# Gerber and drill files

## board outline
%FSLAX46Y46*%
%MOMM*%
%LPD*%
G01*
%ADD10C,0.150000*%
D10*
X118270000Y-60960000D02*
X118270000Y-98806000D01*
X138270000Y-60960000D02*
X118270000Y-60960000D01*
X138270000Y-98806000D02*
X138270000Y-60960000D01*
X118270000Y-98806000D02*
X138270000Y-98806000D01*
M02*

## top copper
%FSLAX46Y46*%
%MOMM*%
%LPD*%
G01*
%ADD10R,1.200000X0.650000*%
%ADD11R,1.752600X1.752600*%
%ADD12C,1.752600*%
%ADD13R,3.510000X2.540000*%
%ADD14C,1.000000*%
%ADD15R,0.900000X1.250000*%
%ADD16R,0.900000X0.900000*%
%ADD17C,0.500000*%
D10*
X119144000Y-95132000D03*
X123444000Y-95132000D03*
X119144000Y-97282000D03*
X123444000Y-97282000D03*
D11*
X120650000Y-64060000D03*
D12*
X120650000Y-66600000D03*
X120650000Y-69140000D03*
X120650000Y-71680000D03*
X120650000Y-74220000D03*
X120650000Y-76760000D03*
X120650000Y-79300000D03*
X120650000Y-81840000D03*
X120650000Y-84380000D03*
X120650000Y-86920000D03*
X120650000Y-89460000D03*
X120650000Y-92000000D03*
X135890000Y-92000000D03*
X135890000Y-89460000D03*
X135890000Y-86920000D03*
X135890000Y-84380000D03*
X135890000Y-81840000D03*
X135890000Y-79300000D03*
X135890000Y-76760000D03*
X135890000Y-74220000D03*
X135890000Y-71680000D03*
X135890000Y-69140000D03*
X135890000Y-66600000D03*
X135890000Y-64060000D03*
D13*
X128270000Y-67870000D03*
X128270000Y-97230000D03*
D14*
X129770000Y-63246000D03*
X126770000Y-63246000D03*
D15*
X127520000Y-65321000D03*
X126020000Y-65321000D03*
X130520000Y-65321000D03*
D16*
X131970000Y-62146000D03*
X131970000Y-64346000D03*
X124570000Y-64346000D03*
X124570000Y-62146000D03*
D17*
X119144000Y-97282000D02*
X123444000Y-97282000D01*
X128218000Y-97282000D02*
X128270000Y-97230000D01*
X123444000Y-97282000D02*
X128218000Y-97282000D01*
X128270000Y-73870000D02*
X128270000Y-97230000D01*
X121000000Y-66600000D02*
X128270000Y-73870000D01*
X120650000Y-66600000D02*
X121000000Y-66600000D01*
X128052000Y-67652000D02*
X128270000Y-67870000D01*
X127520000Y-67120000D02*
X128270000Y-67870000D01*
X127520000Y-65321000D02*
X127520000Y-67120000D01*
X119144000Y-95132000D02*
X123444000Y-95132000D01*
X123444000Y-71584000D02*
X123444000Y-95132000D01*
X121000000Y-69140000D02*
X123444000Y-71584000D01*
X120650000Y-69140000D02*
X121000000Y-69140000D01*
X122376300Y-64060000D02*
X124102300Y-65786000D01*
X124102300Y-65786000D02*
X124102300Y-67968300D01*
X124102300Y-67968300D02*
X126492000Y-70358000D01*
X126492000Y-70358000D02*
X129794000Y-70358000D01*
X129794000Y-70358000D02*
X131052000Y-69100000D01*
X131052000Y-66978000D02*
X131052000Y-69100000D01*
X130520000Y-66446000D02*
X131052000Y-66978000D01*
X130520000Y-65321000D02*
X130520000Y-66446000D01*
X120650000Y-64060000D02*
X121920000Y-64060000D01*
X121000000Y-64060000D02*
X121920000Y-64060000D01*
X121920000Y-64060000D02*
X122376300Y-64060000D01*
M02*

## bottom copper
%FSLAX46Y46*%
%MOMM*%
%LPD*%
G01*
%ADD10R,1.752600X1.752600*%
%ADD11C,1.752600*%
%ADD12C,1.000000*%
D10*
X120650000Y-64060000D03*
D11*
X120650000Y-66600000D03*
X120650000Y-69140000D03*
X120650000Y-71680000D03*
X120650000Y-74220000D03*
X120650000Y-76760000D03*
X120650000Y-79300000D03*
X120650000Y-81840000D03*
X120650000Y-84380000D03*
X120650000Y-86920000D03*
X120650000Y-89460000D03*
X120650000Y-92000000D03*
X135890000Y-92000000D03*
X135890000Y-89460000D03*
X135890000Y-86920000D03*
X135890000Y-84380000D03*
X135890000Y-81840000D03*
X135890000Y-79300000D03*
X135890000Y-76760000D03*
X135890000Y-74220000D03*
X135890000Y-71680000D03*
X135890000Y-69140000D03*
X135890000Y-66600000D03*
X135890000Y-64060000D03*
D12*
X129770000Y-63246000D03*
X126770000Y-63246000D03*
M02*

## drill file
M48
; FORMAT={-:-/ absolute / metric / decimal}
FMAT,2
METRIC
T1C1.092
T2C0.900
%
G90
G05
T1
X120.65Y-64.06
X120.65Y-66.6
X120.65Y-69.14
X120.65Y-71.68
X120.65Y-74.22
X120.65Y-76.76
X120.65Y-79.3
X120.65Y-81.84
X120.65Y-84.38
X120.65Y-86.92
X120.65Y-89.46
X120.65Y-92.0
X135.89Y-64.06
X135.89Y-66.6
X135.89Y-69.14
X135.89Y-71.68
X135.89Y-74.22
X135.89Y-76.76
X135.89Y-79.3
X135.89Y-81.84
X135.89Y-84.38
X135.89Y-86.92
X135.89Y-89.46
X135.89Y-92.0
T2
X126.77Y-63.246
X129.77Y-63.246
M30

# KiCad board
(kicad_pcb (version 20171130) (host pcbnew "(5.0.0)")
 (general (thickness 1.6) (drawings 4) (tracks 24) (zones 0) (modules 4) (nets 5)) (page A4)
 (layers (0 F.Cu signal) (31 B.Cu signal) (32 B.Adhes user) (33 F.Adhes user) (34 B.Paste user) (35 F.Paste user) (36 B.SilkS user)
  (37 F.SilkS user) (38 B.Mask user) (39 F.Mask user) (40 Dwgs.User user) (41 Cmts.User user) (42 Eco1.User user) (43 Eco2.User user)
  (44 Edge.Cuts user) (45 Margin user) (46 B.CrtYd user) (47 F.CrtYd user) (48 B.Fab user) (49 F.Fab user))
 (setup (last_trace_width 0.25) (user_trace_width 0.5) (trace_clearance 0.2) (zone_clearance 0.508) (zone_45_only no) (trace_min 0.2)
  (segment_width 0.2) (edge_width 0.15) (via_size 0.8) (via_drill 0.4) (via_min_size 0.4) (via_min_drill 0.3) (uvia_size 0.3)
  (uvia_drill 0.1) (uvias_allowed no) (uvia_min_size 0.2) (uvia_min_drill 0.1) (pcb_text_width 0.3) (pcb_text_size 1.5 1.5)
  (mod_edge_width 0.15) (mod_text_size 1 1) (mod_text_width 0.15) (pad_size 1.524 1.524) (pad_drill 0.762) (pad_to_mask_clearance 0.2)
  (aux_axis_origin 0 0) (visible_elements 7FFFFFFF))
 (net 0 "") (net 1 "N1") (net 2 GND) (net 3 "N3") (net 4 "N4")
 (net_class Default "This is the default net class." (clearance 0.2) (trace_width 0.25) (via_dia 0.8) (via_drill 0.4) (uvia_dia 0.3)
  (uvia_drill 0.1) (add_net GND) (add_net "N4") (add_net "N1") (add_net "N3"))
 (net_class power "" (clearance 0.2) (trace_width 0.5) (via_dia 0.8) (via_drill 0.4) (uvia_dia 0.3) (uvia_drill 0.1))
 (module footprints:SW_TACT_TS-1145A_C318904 (layer F.Cu) (at 121.294 96.207)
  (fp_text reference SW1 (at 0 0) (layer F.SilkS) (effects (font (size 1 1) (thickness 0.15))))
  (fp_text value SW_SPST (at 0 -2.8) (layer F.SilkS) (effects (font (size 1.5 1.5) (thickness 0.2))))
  (pad 1 smd rect (at -2.15 -1.075) (size 1.2 0.65) (layers F.Cu F.Paste F.Mask) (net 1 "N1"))
  (pad 1 smd rect (at 2.15 -1.075) (size 1.2 0.65) (layers F.Cu F.Paste F.Mask) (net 1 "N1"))
  (pad 2 smd rect (at -2.15 1.075) (size 1.2 0.65) (layers F.Cu F.Paste F.Mask) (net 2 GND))
  (pad 2 smd rect (at 2.15 1.075) (size 1.2 0.65) (layers F.Cu F.Paste F.Mask) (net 2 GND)))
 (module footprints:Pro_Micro (layer F.Cu) (at 128.27 76.506)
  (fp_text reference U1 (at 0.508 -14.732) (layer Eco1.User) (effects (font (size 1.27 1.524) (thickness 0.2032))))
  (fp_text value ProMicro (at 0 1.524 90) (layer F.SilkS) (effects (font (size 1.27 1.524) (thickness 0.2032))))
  (pad 1 thru_hole rect (at -7.62 -12.446 270) (size 1.7526 1.7526) (drill 1.0922) (layers *.Cu *.SilkS *.Mask) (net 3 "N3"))
  (pad 2 thru_hole circle (at -7.62 -9.906 270) (size 1.7526 1.7526) (drill 1.0922) (layers *.Cu *.SilkS *.Mask) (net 2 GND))
  (pad 3 thru_hole circle (at -7.62 -7.366 270) (size 1.7526 1.7526) (drill 1.0922) (layers *.Cu *.SilkS *.Mask) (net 1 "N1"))
  (pad 4 thru_hole circle (at -7.62 -4.826 270) (size 1.7526 1.7526) (drill 1.0922) (layers *.Cu *.SilkS *.Mask))
  (pad 5 thru_hole circle (at -7.62 -2.286 270) (size 1.7526 1.7526) (drill 1.0922) (layers *.Cu *.SilkS *.Mask))
  (pad 6 thru_hole circle (at -7.62 0.254 270) (size 1.7526 1.7526) (drill 1.0922) (layers *.Cu *.SilkS *.Mask))
  (pad 7 thru_hole circle (at -7.62 2.794 270) (size 1.7526 1.7526) (drill 1.0922) (layers *.Cu *.SilkS *.Mask))
  (pad 8 thru_hole circle (at -7.62 5.334 270) (size 1.7526 1.7526) (drill 1.0922) (layers *.Cu *.SilkS *.Mask))
  (pad 9 thru_hole circle (at -7.62 7.874 270) (size 1.7526 1.7526) (drill 1.0922) (layers *.Cu *.SilkS *.Mask))
  (pad 10 thru_hole circle (at -7.62 10.414 270) (size 1.7526 1.7526) (drill 1.0922) (layers *.Cu *.SilkS *.Mask))
  (pad 11 thru_hole circle (at -7.62 12.954 270) (size 1.7526 1.7526) (drill 1.0922) (layers *.Cu *.SilkS *.Mask))
  (pad 12 thru_hole circle (at -7.62 15.494 270) (size 1.7526 1.7526) (drill 1.0922) (layers *.Cu *.SilkS *.Mask))
  (pad 24 thru_hole circle (at 7.62 15.494 270) (size 1.7526 1.7526) (drill 1.0922) (layers *.Cu *.SilkS *.Mask))
  (pad 23 thru_hole circle (at 7.62 12.954 270) (size 1.7526 1.7526) (drill 1.0922) (layers *.Cu *.SilkS *.Mask))
  (pad 22 thru_hole circle (at 7.62 10.414 270) (size 1.7526 1.7526) (drill 1.0922) (layers *.Cu *.SilkS *.Mask))
  (pad 21 thru_hole circle (at 7.62 7.874 270) (size 1.7526 1.7526) (drill 1.0922) (layers *.Cu *.SilkS *.Mask))
  (pad 20 thru_hole circle (at 7.62 5.334 270) (size 1.7526 1.7526) (drill 1.0922) (layers *.Cu *.SilkS *.Mask))
  (pad 19 thru_hole circle (at 7.62 2.794 270) (size 1.7526 1.7526) (drill 1.0922) (layers *.Cu *.SilkS *.Mask))
  (pad 18 thru_hole circle (at 7.62 0.254 270) (size 1.7526 1.7526) (drill 1.0922) (layers *.Cu *.SilkS *.Mask))
  (pad 17 thru_hole circle (at 7.62 -2.286 270) (size 1.7526 1.7526) (drill 1.0922) (layers *.Cu *.SilkS *.Mask))
  (pad 16 thru_hole circle (at 7.62 -4.826 270) (size 1.7526 1.7526) (drill 1.0922) (layers *.Cu *.SilkS *.Mask))
  (pad 15 thru_hole circle (at 7.62 -7.366 270) (size 1.7526 1.7526) (drill 1.0922) (layers *.Cu *.SilkS *.Mask))
  (pad 14 thru_hole circle (at 7.62 -9.906 270) (size 1.7526 1.7526) (drill 1.0922) (layers *.Cu *.SilkS *.Mask))
  (pad 13 thru_hole circle (at 7.62 -12.446 270) (size 1.7526 1.7526) (drill 1.0922) (layers *.Cu *.SilkS *.Mask)))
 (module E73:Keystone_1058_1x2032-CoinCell (layer F.Cu) (at 128.27 82.55 270)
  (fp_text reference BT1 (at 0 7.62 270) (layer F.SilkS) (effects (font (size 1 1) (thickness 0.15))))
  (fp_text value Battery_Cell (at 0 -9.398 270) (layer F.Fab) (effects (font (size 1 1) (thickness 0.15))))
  (pad 1 smd rect (at -14.68 0 270) (size 2.54 3.51) (layers F.Cu F.Paste F.Mask) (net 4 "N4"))
  (pad 2 smd rect (at 14.68 0 270) (size 2.54 3.51) (layers F.Cu F.Paste F.Mask) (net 2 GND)))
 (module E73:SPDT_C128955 (layer F.Cu) (at 128.27 63.246)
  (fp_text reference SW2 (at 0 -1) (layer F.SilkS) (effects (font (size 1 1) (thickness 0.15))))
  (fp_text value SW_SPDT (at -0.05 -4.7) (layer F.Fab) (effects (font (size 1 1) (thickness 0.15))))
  (pad "" np_thru_hole circle (at 1.5 0) (size 1 1) (drill 0.9) (layers *.Cu *.Mask))
  (pad "" np_thru_hole circle (at -1.5 0) (size 1 1) (drill 0.9) (layers *.Cu *.Mask))
  (pad 2 smd rect (at -0.75 2.075) (size 0.9 1.25) (layers F.Cu F.Paste F.Mask) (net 4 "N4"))
  (pad 3 smd rect (at -2.25 2.075) (size 0.9 1.25) (layers F.Cu F.Paste F.Mask))
  (pad 1 smd rect (at 2.25 2.075) (size 0.9 1.25) (layers F.Cu F.Paste F.Mask) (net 3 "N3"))
  (pad 0 smd rect (at 3.7 -1.1) (size 0.9 0.9) (layers F.Cu F.Paste F.Mask))
  (pad 0 smd rect (at 3.7 1.1) (size 0.9 0.9) (layers F.Cu F.Paste F.Mask))
  (pad 0 smd rect (at -3.7 1.1) (size 0.9 0.9) (layers F.Cu F.Paste F.Mask))
  (pad 0 smd rect (at -3.7 -1.1) (size 0.9 0.9) (layers F.Cu F.Paste F.Mask)))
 (gr_line (start 118.27 60.96) (end 118.27 98.806) (layer Edge.Cuts) (width 0.15))
 (gr_line (start 138.27 60.96) (end 118.27 60.96) (layer Edge.Cuts) (width 0.15))
 (gr_line (start 138.27 98.806) (end 138.27 60.96) (layer Edge.Cuts) (width 0.15))
 (gr_line (start 118.27 98.806) (end 138.27 98.806) (layer Edge.Cuts) (width 0.15))
 (segment (start 119.144 97.282) (end 123.444 97.282) (width 0.5) (layer F.Cu) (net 2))
 (segment (start 128.218 97.282) (end 128.27 97.23) (width 0.5) (layer F.Cu) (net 2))
 (segment (start 123.444 97.282) (end 128.218 97.282) (width 0.5) (layer F.Cu) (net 2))
 (segment (start 128.27 73.87) (end 128.27 97.23) (width 0.5) (layer F.Cu) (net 2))
 (segment (start 121 66.6) (end 128.27 73.87) (width 0.5) (layer F.Cu) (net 2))
 (segment (start 120.65 66.6) (end 121 66.6) (width 0.5) (layer F.Cu) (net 2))
 (segment (start 128.052 67.652) (end 128.27 67.87) (width 0.5) (layer F.Cu) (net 4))
 (segment (start 127.52 67.12) (end 128.27 67.87) (width 0.5) (layer F.Cu) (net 4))
 (segment (start 127.52 65.321) (end 127.52 67.12) (width 0.5) (layer F.Cu) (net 4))
 (segment (start 119.144 95.132) (end 123.444 95.132) (width 0.5) (layer F.Cu) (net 1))
 (segment (start 123.444 71.584) (end 123.444 95.132) (width 0.5) (layer F.Cu) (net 1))
 (segment (start 121 69.14) (end 123.444 71.584) (width 0.5) (layer F.Cu) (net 1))
 (segment (start 120.65 69.14) (end 121 69.14) (width 0.5) (layer F.Cu) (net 1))
 (segment (start 122.3763 64.06) (end 124.1023 65.786) (width 0.5) (layer F.Cu) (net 3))
 (segment (start 124.1023 65.786) (end 124.1023 67.9683) (width 0.5) (layer F.Cu) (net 3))
 (segment (start 124.1023 67.9683) (end 126.492 70.358) (width 0.5) (layer F.Cu) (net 3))
 (segment (start 126.492 70.358) (end 129.794 70.358) (width 0.5) (layer F.Cu) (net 3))
 (segment (start 129.794 70.358) (end 131.052 69.1) (width 0.5) (layer F.Cu) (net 3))
 (segment (start 131.052 66.978) (end 131.052 69.1) (width 0.5) (layer F.Cu) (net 3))
 (segment (start 130.52 66.446) (end 131.052 66.978) (width 0.5) (layer F.Cu) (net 3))
 (segment (start 130.52 65.321) (end 130.52 66.446) (width 0.5) (layer F.Cu) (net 3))
 (segment (start 120.65 64.06) (end 121.92 64.06) (width 0.5) (layer F.Cu) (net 3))
 (segment (start 121 64.06) (end 121.92 64.06) (width 0.5) (layer F.Cu) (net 3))
 (segment (start 121.92 64.06) (end 122.3763 64.06) (width 0.5) (layer F.Cu) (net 3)))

